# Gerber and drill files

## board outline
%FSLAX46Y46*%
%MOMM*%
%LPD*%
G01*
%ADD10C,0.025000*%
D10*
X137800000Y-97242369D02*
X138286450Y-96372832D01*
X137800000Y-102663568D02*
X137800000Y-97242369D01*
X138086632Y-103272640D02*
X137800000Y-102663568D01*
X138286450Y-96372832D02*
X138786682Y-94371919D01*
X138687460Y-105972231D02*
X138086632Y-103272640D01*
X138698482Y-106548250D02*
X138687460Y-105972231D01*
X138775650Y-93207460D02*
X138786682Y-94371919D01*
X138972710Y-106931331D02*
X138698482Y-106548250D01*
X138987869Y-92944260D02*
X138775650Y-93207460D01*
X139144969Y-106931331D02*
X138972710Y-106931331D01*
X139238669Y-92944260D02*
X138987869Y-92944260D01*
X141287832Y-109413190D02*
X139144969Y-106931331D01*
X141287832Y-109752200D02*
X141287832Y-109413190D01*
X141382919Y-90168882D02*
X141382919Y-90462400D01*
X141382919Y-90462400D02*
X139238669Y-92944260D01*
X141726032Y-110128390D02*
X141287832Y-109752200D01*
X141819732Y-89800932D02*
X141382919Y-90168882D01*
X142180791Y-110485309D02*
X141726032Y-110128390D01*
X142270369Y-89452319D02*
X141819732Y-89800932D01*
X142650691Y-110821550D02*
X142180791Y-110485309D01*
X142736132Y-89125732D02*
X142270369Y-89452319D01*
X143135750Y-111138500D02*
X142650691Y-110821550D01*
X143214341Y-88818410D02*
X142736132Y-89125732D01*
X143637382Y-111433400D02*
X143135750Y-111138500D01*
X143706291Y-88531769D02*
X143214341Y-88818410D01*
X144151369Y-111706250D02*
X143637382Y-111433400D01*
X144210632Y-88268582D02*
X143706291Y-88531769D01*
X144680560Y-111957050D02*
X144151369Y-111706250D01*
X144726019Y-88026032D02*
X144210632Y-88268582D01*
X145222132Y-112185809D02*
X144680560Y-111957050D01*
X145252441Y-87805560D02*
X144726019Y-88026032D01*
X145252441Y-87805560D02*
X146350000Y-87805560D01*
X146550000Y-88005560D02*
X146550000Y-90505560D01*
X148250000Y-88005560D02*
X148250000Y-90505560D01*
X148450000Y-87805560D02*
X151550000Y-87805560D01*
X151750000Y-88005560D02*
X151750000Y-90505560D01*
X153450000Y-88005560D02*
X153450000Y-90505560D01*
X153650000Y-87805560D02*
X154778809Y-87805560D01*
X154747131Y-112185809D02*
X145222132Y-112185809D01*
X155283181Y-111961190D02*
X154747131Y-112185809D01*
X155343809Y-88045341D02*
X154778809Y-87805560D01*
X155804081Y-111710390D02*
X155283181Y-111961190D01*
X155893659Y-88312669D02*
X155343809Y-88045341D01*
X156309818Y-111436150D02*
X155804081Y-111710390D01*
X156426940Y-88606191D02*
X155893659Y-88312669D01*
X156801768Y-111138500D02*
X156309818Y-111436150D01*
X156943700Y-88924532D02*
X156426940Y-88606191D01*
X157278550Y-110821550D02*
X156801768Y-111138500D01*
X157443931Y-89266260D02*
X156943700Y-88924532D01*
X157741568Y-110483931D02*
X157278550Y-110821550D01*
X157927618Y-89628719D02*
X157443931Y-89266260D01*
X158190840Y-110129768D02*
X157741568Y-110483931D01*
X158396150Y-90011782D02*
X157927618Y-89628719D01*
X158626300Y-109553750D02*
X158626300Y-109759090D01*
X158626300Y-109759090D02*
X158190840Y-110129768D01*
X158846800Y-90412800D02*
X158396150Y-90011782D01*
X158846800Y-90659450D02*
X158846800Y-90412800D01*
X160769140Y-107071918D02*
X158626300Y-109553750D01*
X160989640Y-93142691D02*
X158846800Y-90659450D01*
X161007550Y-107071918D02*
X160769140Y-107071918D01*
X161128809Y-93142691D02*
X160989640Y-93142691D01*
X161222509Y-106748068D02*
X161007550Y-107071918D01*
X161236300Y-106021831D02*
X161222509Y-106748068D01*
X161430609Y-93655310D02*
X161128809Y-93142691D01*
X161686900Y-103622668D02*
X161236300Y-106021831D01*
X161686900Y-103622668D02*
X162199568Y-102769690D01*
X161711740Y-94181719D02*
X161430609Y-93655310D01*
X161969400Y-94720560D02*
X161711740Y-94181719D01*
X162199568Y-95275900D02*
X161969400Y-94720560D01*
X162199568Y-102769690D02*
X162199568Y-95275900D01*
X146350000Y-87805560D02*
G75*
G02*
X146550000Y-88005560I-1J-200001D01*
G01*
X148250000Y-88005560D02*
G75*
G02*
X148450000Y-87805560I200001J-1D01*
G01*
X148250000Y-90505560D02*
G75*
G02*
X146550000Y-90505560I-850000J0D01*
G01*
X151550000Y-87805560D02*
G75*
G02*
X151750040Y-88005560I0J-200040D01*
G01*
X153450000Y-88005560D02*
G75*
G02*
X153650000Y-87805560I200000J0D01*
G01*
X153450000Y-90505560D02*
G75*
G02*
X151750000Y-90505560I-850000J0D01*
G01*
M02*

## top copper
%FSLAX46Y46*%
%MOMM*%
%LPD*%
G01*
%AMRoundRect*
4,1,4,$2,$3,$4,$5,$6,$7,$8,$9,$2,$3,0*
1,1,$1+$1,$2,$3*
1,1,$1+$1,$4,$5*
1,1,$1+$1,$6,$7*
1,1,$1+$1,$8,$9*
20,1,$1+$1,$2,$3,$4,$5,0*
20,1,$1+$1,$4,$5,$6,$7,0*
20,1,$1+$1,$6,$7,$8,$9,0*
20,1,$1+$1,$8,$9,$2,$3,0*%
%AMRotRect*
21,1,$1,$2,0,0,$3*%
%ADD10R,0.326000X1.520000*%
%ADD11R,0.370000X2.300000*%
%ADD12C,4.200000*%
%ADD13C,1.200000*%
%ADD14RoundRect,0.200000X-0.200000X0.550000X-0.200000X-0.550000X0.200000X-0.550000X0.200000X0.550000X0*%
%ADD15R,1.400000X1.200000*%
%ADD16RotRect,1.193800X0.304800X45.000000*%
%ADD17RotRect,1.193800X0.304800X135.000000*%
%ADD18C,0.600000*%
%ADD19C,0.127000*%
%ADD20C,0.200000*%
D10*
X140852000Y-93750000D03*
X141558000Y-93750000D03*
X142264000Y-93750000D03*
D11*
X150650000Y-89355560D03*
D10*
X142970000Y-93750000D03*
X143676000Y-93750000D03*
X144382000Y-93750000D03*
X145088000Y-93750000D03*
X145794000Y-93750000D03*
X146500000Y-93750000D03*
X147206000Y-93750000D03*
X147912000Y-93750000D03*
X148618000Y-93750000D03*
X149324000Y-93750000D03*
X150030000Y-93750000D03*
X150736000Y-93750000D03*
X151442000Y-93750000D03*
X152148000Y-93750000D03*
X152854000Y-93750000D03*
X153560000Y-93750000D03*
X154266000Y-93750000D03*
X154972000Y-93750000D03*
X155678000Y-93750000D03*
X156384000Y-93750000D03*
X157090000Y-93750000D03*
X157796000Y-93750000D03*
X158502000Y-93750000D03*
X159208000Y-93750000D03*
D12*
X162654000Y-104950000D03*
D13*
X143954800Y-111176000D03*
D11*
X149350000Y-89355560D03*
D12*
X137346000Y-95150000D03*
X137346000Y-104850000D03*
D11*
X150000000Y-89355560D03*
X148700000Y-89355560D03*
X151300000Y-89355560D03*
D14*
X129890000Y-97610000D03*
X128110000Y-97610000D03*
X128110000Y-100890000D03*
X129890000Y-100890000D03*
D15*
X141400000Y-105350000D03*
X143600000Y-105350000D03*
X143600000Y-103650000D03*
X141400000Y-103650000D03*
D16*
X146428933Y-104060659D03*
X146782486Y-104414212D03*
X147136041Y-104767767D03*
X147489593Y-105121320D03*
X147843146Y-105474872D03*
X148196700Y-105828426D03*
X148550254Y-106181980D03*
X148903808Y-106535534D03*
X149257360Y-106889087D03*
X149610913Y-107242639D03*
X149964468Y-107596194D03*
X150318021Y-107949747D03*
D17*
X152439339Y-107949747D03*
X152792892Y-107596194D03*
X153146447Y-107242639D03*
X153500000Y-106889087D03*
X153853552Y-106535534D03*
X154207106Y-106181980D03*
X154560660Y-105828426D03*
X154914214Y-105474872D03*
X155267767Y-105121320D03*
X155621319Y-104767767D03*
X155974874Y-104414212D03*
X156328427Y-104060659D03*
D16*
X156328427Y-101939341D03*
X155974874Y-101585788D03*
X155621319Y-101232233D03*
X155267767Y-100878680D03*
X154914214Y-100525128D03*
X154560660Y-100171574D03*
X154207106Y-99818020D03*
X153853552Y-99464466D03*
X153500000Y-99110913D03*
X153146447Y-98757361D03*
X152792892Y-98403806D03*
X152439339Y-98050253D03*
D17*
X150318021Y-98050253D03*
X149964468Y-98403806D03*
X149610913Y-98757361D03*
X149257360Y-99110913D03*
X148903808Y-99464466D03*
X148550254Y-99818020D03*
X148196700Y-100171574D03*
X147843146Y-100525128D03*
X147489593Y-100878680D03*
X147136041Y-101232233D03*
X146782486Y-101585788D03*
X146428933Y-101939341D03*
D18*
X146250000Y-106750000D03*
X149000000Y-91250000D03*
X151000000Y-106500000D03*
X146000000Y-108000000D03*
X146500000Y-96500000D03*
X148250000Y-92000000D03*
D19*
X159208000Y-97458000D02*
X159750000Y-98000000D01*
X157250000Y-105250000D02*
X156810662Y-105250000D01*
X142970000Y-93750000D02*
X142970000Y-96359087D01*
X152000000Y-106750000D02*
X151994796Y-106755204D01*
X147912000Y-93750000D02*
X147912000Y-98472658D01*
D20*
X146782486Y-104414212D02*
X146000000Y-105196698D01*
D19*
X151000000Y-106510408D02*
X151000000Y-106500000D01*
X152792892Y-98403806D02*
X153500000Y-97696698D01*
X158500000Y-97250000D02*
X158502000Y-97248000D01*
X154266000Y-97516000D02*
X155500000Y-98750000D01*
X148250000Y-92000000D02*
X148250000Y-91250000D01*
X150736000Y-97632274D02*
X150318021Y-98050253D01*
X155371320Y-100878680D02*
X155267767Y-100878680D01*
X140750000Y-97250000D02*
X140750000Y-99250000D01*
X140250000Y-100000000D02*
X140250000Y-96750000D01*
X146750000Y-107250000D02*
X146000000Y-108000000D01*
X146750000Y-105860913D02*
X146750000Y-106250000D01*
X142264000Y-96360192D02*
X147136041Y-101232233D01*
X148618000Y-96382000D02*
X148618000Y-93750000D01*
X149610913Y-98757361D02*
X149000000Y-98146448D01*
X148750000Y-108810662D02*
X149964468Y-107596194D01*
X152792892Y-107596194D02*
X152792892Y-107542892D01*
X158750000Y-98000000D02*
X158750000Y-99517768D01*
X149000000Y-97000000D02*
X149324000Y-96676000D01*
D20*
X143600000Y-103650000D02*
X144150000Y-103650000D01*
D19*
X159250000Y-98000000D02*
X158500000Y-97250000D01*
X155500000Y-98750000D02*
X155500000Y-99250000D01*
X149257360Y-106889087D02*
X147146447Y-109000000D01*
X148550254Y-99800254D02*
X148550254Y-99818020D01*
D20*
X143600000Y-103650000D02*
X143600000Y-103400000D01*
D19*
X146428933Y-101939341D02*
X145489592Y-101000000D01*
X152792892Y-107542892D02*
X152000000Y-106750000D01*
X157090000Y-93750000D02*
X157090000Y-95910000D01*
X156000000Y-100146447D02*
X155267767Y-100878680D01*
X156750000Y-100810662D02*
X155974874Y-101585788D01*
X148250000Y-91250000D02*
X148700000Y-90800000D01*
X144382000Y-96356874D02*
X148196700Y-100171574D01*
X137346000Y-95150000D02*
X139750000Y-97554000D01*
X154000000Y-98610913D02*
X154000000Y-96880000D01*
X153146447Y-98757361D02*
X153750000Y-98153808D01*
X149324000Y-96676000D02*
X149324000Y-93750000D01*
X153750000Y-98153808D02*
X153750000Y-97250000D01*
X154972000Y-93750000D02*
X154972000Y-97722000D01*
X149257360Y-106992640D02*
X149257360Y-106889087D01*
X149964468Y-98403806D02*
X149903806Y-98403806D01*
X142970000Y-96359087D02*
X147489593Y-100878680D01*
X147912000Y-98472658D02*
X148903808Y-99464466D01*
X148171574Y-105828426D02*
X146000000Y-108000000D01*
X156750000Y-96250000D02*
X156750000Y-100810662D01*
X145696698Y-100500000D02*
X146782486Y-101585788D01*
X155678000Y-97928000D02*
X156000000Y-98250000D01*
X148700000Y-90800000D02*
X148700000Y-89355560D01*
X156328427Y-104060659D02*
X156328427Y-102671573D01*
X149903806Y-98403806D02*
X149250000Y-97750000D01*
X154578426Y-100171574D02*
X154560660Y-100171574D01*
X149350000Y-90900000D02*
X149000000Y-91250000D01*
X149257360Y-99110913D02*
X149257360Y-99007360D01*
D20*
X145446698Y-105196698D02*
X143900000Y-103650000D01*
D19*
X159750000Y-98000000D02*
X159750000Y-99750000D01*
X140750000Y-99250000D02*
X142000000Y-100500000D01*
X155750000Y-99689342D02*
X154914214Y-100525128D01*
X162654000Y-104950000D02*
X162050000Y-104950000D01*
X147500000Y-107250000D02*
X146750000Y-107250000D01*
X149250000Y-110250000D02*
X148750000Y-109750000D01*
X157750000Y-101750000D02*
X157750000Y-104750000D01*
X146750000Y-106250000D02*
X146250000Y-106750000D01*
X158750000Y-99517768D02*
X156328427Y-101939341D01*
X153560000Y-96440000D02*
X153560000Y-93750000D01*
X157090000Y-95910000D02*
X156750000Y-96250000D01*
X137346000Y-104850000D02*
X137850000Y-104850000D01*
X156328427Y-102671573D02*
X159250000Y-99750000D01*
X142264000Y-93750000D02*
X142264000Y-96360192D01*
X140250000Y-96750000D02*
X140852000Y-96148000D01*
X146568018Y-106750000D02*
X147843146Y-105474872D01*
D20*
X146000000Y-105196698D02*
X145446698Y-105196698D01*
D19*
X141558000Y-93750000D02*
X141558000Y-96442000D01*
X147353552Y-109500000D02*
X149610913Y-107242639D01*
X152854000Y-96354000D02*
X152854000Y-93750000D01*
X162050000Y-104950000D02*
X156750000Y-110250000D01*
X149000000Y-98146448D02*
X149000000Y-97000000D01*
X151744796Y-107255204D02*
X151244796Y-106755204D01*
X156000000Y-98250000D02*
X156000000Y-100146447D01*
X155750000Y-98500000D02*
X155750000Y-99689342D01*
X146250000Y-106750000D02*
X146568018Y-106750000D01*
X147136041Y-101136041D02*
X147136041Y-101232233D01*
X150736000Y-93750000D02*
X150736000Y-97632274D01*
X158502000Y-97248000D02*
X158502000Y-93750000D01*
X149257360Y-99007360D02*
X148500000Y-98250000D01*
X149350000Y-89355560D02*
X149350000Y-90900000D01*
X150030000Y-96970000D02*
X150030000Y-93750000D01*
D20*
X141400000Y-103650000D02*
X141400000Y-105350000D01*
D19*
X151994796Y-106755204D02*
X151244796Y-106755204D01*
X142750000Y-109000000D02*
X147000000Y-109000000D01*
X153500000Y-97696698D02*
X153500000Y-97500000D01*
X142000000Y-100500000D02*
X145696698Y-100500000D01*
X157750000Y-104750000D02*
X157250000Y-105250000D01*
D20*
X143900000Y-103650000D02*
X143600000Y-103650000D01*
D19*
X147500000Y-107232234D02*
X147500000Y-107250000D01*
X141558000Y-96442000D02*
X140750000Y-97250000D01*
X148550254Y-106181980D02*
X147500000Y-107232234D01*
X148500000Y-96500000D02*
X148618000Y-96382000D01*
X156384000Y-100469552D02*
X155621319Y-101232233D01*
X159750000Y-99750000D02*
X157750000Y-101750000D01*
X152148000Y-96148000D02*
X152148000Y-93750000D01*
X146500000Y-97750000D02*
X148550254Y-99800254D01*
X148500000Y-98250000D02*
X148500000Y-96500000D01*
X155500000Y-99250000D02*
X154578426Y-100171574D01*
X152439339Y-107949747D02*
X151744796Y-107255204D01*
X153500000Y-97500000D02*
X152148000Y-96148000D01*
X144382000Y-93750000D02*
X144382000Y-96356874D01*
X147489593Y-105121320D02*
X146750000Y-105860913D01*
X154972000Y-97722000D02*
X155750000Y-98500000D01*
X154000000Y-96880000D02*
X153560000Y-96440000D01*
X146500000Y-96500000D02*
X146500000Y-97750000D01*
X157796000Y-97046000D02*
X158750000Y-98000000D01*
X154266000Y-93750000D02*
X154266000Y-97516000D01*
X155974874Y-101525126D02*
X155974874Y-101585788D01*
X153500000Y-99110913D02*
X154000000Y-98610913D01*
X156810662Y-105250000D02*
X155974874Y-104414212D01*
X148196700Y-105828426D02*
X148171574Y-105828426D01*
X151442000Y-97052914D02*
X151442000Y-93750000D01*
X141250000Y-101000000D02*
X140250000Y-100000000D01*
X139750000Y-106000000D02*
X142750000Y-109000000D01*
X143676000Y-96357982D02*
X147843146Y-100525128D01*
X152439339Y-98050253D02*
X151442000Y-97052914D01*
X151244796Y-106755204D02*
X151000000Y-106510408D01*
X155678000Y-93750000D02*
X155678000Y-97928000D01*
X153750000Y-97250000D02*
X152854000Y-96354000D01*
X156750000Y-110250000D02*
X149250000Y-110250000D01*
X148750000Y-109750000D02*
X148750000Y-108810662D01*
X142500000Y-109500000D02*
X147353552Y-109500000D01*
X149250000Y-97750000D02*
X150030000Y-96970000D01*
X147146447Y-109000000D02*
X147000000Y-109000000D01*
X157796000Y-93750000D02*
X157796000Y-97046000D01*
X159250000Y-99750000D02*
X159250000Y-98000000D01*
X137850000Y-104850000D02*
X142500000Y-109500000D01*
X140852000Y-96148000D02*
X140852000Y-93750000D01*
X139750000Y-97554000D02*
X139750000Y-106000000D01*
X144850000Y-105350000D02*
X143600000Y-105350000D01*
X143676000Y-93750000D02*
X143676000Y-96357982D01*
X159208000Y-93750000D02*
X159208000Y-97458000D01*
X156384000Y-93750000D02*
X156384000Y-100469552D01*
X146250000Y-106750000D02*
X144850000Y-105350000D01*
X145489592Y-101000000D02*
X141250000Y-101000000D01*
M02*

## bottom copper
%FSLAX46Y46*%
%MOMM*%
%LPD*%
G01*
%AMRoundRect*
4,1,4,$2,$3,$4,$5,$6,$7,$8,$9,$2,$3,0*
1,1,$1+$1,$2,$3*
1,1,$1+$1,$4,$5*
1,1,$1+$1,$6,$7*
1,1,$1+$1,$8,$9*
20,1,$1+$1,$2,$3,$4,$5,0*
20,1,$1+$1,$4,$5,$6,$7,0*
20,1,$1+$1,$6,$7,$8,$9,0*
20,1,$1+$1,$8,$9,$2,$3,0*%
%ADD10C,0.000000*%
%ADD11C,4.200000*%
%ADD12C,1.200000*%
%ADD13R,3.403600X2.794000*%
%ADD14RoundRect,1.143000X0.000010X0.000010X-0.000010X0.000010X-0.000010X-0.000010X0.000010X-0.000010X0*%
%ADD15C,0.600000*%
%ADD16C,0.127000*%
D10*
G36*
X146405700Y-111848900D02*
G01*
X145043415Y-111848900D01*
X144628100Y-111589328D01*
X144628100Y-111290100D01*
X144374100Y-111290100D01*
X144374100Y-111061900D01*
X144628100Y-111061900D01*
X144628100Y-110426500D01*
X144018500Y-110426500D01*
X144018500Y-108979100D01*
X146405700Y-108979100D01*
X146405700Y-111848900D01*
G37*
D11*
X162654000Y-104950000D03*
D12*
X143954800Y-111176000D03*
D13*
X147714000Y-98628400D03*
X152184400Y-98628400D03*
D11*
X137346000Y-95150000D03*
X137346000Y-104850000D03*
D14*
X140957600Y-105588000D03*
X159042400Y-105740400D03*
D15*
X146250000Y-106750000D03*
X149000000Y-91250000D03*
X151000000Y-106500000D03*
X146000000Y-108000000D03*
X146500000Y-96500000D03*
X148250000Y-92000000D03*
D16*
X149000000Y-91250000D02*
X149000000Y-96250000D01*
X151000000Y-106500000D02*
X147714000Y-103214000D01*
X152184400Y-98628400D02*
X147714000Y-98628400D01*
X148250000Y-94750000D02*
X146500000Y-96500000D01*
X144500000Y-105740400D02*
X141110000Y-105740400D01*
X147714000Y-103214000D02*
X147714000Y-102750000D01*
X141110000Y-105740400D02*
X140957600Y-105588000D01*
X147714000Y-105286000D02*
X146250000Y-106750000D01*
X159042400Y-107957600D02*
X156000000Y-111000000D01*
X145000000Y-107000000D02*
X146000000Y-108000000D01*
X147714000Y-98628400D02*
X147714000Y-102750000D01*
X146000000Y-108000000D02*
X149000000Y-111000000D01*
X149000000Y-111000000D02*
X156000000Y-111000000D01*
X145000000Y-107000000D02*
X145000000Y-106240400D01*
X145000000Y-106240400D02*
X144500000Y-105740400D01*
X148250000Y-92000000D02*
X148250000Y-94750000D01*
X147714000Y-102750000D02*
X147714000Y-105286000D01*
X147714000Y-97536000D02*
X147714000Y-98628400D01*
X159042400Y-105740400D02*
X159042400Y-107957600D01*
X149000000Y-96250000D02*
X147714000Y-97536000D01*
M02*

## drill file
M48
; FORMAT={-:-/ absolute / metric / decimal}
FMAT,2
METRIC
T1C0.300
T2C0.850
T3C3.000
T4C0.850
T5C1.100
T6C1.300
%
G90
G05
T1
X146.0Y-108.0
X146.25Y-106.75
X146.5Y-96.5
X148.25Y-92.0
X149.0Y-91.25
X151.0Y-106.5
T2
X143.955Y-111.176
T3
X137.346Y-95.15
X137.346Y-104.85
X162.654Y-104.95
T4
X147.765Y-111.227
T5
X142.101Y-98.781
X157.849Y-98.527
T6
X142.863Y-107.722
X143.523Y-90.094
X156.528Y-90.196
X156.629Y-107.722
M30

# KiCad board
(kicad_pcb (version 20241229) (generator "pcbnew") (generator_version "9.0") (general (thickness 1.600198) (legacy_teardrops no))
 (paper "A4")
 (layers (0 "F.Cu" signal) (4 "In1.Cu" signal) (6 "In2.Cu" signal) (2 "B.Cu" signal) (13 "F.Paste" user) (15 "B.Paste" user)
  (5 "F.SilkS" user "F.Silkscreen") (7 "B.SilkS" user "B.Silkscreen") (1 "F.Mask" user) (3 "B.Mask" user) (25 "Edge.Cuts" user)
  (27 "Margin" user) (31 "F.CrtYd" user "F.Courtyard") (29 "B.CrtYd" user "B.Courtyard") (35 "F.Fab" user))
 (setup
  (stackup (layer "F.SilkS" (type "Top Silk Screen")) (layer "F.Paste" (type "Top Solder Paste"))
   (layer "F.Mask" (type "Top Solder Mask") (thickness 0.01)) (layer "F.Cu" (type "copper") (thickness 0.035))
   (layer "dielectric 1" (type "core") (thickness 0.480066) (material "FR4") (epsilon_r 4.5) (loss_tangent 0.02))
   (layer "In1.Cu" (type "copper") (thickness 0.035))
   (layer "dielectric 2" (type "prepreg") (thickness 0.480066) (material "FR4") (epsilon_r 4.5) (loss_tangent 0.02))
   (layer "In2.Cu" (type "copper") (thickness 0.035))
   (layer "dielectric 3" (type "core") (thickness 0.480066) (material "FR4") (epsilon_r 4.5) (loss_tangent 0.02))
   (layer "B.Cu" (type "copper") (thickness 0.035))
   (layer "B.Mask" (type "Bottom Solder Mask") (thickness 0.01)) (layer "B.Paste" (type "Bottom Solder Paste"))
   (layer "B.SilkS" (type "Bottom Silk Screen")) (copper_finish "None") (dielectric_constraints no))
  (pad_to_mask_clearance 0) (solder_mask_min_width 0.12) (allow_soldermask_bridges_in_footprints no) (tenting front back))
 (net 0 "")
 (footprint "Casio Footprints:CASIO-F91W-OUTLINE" (layer "F.Cu") (at 150 100)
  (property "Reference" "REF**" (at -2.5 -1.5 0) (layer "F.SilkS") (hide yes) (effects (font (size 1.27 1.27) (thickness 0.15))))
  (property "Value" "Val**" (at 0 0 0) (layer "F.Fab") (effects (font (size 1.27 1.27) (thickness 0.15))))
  (fp_poly
   (pts (xy -3.5943 11.8489) (xy -4.956585 11.8489) (xy -5.3719 11.589328) (xy -5.3719 11.2901) (xy -5.6259 11.2901) (xy -5.6259 11.0619)
    (xy -5.3719 11.0619) (xy -5.3719 10.4265) (xy -5.9815 10.4265) (xy -5.9815 8.9791) (xy -3.5943 8.9791))
   (stroke (width 0) (type solid)) (fill yes) (layer "B.Cu"))
  (fp_line (start -12.2 -2.757631) (end -11.71355 -3.627168) (stroke (width 0.025) (type solid)) (layer "Edge.Cuts"))
  (fp_line (start -12.2 2.663568) (end -12.2 -2.757631) (stroke (width 0.025) (type solid)) (layer "Edge.Cuts"))
  (fp_line (start -11.913368 3.27264) (end -12.2 2.663568) (stroke (width 0.025) (type solid)) (layer "Edge.Cuts"))
  (fp_line (start -11.71355 -3.627168) (end -11.213318 -5.628081) (stroke (width 0.025) (type solid)) (layer "Edge.Cuts"))
  (fp_line (start -11.31254 5.972231) (end -11.913368 3.27264) (stroke (width 0.025) (type solid)) (layer "Edge.Cuts"))
  (fp_line (start -11.301518 6.54825) (end -11.31254 5.972231) (stroke (width 0.025) (type solid)) (layer "Edge.Cuts"))
  (fp_line (start -11.22435 -6.79254) (end -11.213318 -5.628081) (stroke (width 0.025) (type solid)) (layer "Edge.Cuts"))
  (fp_line (start -11.02729 6.931331) (end -11.301518 6.54825) (stroke (width 0.025) (type solid)) (layer "Edge.Cuts"))
  (fp_line (start -11.012131 -7.05574) (end -11.22435 -6.79254) (stroke (width 0.025) (type solid)) (layer "Edge.Cuts"))
  (fp_line (start -10.855031 6.931331) (end -11.02729 6.931331) (stroke (width 0.025) (type solid)) (layer "Edge.Cuts"))
  (fp_line (start -10.761331 -7.05574) (end -11.012131 -7.05574) (stroke (width 0.025) (type solid)) (layer "Edge.Cuts"))
  (fp_line (start -8.712168 9.41319) (end -10.855031 6.931331) (stroke (width 0.025) (type solid)) (layer "Edge.Cuts"))
  (fp_line (start -8.712168 9.7522) (end -8.712168 9.41319) (stroke (width 0.025) (type solid)) (layer "Edge.Cuts"))
  (fp_line (start -8.617081 -9.831118) (end -8.617081 -9.5376) (stroke (width 0.025) (type solid)) (layer "Edge.Cuts"))
  (fp_line (start -8.617081 -9.5376) (end -10.761331 -7.05574) (stroke (width 0.025) (type solid)) (layer "Edge.Cuts"))
  (fp_line (start -8.273968 10.12839) (end -8.712168 9.7522) (stroke (width 0.025) (type solid)) (layer "Edge.Cuts"))
  (fp_line (start -8.180268 -10.199068) (end -8.617081 -9.831118) (stroke (width 0.025) (type solid)) (layer "Edge.Cuts"))
  (fp_line (start -7.819209 10.485309) (end -8.273968 10.12839) (stroke (width 0.025) (type solid)) (layer "Edge.Cuts"))
  (fp_line (start -7.729631 -10.547681) (end -8.180268 -10.199068) (stroke (width 0.025) (type solid)) (layer "Edge.Cuts"))
  (fp_line (start -7.349309 10.82155) (end -7.819209 10.485309) (stroke (width 0.025) (type solid)) (layer "Edge.Cuts"))
  (fp_line (start -7.263868 -10.874268) (end -7.729631 -10.547681) (stroke (width 0.025) (type solid)) (layer "Edge.Cuts"))
  (fp_line (start -6.86425 11.1385) (end -7.349309 10.82155) (stroke (width 0.025) (type solid)) (layer "Edge.Cuts"))
  (fp_line (start -6.785659 -11.18159) (end -7.263868 -10.874268) (stroke (width 0.025) (type solid)) (layer "Edge.Cuts"))
  (fp_line (start -6.362618 11.4334) (end -6.86425 11.1385) (stroke (width 0.025) (type solid)) (layer "Edge.Cuts"))
  (fp_line (start -6.293709 -11.468231) (end -6.785659 -11.18159) (stroke (width 0.025) (type solid)) (layer "Edge.Cuts"))
  (fp_line (start -5.848631 11.70625) (end -6.362618 11.4334) (stroke (width 0.025) (type solid)) (layer "Edge.Cuts"))
  (fp_line (start -5.789368 -11.731418) (end -6.293709 -11.468231) (stroke (width 0.025) (type solid)) (layer "Edge.Cuts"))
  (fp_line (start -5.31944 11.95705) (end -5.848631 11.70625) (stroke (width 0.025) (type solid)) (layer "Edge.Cuts"))
  (fp_line (start -5.273981 -11.973968) (end -5.789368 -11.731418) (stroke (width 0.025) (type solid)) (layer "Edge.Cuts"))
  (fp_line (start -4.777868 12.185809) (end -5.31944 11.95705) (stroke (width 0.025) (type solid)) (layer "Edge.Cuts"))
  (fp_line (start -4.747559 -12.19444) (end -5.273981 -11.973968) (stroke (width 0.025) (type solid)) (layer "Edge.Cuts"))
  (fp_line (start -4.747559 -12.19444) (end -3.65 -12.19444) (stroke (width 0.025) (type solid)) (layer "Edge.Cuts"))
  (fp_line (start -3.45 -11.99444) (end -3.45 -9.49444) (stroke (width 0.025) (type solid)) (layer "Edge.Cuts"))
  (fp_line (start -1.75 -11.99444) (end -1.75 -9.49444) (stroke (width 0.025) (type solid)) (layer "Edge.Cuts"))
  (fp_line (start -1.55 -12.19444) (end 1.55 -12.19444) (stroke (width 0.025) (type solid)) (layer "Edge.Cuts"))
  (fp_line (start 1.75 -11.99444) (end 1.75 -9.49444) (stroke (width 0.025) (type solid)) (layer "Edge.Cuts"))
  (fp_line (start 3.45 -11.99444) (end 3.45 -9.49444) (stroke (width 0.025) (type solid)) (layer "Edge.Cuts"))
  (fp_line (start 3.65 -12.19444) (end 4.778809 -12.19444) (stroke (width 0.025) (type solid)) (layer "Edge.Cuts"))
  (fp_line (start 4.747131 12.185809) (end -4.777868 12.185809) (stroke (width 0.025) (type solid)) (layer "Edge.Cuts"))
  (fp_line (start 5.283181 11.96119) (end 4.747131 12.185809) (stroke (width 0.025) (type solid)) (layer "Edge.Cuts"))
  (fp_line (start 5.343809 -11.954659) (end 4.778809 -12.19444) (stroke (width 0.025) (type solid)) (layer "Edge.Cuts"))
  (fp_line (start 5.804081 11.71039) (end 5.283181 11.96119) (stroke (width 0.025) (type solid)) (layer "Edge.Cuts"))
  (fp_line (start 5.893659 -11.687331) (end 5.343809 -11.954659) (stroke (width 0.025) (type solid)) (layer "Edge.Cuts"))
  (fp_line (start 6.309818 11.43615) (end 5.804081 11.71039) (stroke (width 0.025) (type solid)) (layer "Edge.Cuts"))
  (fp_line (start 6.42694 -11.393809) (end 5.893659 -11.687331) (stroke (width 0.025) (type solid)) (layer "Edge.Cuts"))
  (fp_line (start 6.801768 11.1385) (end 6.309818 11.43615) (stroke (width 0.025) (type solid)) (layer "Edge.Cuts"))
  (fp_line (start 6.9437 -11.075468) (end 6.42694 -11.393809) (stroke (width 0.025) (type solid)) (layer "Edge.Cuts"))
  (fp_line (start 7.27855 10.82155) (end 6.801768 11.1385) (stroke (width 0.025) (type solid)) (layer "Edge.Cuts"))
  (fp_line (start 7.443931 -10.73374) (end 6.9437 -11.075468) (stroke (width 0.025) (type solid)) (layer "Edge.Cuts"))
  (fp_line (start 7.741568 10.483931) (end 7.27855 10.82155) (stroke (width 0.025) (type solid)) (layer "Edge.Cuts"))
  (fp_line (start 7.927618 -10.371281) (end 7.443931 -10.73374) (stroke (width 0.025) (type solid)) (layer "Edge.Cuts"))
  (fp_line (start 8.19084 10.129768) (end 7.741568 10.483931) (stroke (width 0.025) (type solid)) (layer "Edge.Cuts"))
  (fp_line (start 8.39615 -9.988218) (end 7.927618 -10.371281) (stroke (width 0.025) (type solid)) (layer "Edge.Cuts"))
  (fp_line (start 8.6263 9.55375) (end 8.6263 9.75909) (stroke (width 0.025) (type solid)) (layer "Edge.Cuts"))
  (fp_line (start 8.6263 9.75909) (end 8.19084 10.129768) (stroke (width 0.025) (type solid)) (layer "Edge.Cuts"))
  (fp_line (start 8.8468 -9.5872) (end 8.39615 -9.988218) (stroke (width 0.025) (type solid)) (layer "Edge.Cuts"))
  (fp_line (start 8.8468 -9.34055) (end 8.8468 -9.5872) (stroke (width 0.025) (type solid)) (layer "Edge.Cuts"))
  (fp_line (start 10.76914 7.071918) (end 8.6263 9.55375) (stroke (width 0.025) (type solid)) (layer "Edge.Cuts"))
  (fp_line (start 10.98964 -6.857309) (end 8.8468 -9.34055) (stroke (width 0.025) (type solid)) (layer "Edge.Cuts"))
  (fp_line (start 11.00755 7.071918) (end 10.76914 7.071918) (stroke (width 0.025) (type solid)) (layer "Edge.Cuts"))
  (fp_line (start 11.128809 -6.857309) (end 10.98964 -6.857309) (stroke (width 0.025) (type solid)) (layer "Edge.Cuts"))
  (fp_line (start 11.222509 6.748068) (end 11.00755 7.071918) (stroke (width 0.025) (type solid)) (layer "Edge.Cuts"))
  (fp_line (start 11.2363 6.021831) (end 11.222509 6.748068) (stroke (width 0.025) (type solid)) (layer "Edge.Cuts"))
  (fp_line (start 11.430609 -6.34469) (end 11.128809 -6.857309) (stroke (width 0.025) (type solid)) (layer "Edge.Cuts"))
  (fp_line (start 11.6869 3.622668) (end 11.2363 6.021831) (stroke (width 0.025) (type solid)) (layer "Edge.Cuts"))
  (fp_line (start 11.6869 3.622668) (end 12.199568 2.76969) (stroke (width 0.025) (type solid)) (layer "Edge.Cuts"))
  (fp_line (start 11.71174 -5.818281) (end 11.430609 -6.34469) (stroke (width 0.025) (type solid)) (layer "Edge.Cuts"))
  (fp_line (start 11.9694 -5.27944) (end 11.71174 -5.818281) (stroke (width 0.025) (type solid)) (layer "Edge.Cuts"))
  (fp_line (start 12.199568 -4.7241) (end 11.9694 -5.27944) (stroke (width 0.025) (type solid)) (layer "Edge.Cuts"))
  (fp_line (start 12.199568 2.76969) (end 12.199568 -4.7241) (stroke (width 0.025) (type solid)) (layer "Edge.Cuts"))
  (fp_arc (start -3.65 -12.19444) (mid -3.508579 -12.135861) (end -3.45 -11.99444) (stroke (width 0.025) (type solid)) (layer "Edge.Cuts"))
  (fp_arc (start -1.75 -11.99444) (mid -1.691421 -12.135861) (end -1.55 -12.19444) (stroke (width 0.025) (type solid)) (layer "Edge.Cuts"))
  (fp_arc (start -1.75 -9.49444) (mid -2.6 -8.64444) (end -3.45 -9.49444) (stroke (width 0.025) (type solid)) (layer "Edge.Cuts"))
  (fp_arc (start 1.55 -12.19444) (mid 1.691421 -12.135861) (end 1.75 -11.99444) (stroke (width 0.025) (type solid)) (layer "Edge.Cuts"))
  (fp_arc (start 3.45 -11.99444) (mid 3.508579 -12.135861) (end 3.65 -12.19444) (stroke (width 0.025) (type solid)) (layer "Edge.Cuts"))
  (fp_arc (start 3.45 -9.49444) (mid 2.6 -8.64444) (end 1.75 -9.49444) (stroke (width 0.025) (type solid)) (layer "Edge.Cuts"))
  (pad "" np_thru_hole circle (at -7.8994 -1.2192) (size 1.1 1.1) (drill 1.1) (layers "*.Cu" "*.Mask"))
  (pad "" np_thru_hole circle (at -7.1374 7.7216) (size 1.3 1.3) (drill 1.3) (layers "*.Cu" "*.Mask"))
  (pad "" np_thru_hole circle (at -6.477 -9.906) (size 1.3 1.3) (drill 1.3) (layers "*.Cu" "*.Mask"))
  (pad "" np_thru_hole circle (at -2.2352 11.2268) (size 0.85 0.85) (drill 0.85) (layers "*.Cu" "*.Mask"))
  (pad "" np_thru_hole circle (at 6.5278 -9.8044) (size 1.3 1.3) (drill 1.3) (layers "*.Cu" "*.Mask"))
  (pad "" np_thru_hole circle (at 6.6294 7.7216) (size 1.3 1.3) (drill 1.3) (layers "*.Cu" "*.Mask"))
  (pad "" np_thru_hole circle (at 7.8486 -1.4732) (size 1.1 1.1) (drill 1.1) (layers "*.Cu" "*.Mask"))
  (pad "1" smd rect (at -9.148 -6.25) (size 0.326 1.52) (layers "F.Cu" "F.Mask") (solder_mask_margin 0.0635))
  (pad "2" smd rect (at -8.442 -6.25) (size 0.326 1.52) (layers "F.Cu" "F.Mask") (solder_mask_margin 0.0635))
  (pad "3" smd rect (at -7.736 -6.25) (size 0.326 1.52) (layers "F.Cu" "F.Mask") (solder_mask_margin 0.0635))
  (pad "3V3" smd rect (at 0.65 -10.64444 90) (size 2.3 0.37) (layers "F.Cu" "F.Mask") (solder_mask_margin 0.0635))
  (pad "4" smd rect (at -7.03 -6.25) (size 0.326 1.52) (layers "F.Cu" "F.Mask") (solder_mask_margin 0.0635))
  (pad "5" smd rect (at -6.324 -6.25) (size 0.326 1.52) (layers "F.Cu" "F.Mask") (solder_mask_margin 0.0635))
  (pad "6" smd rect (at -5.618 -6.25) (size 0.326 1.52) (layers "F.Cu" "F.Mask") (solder_mask_margin 0.0635))
  (pad "7" smd rect (at -4.912 -6.25) (size 0.326 1.52) (layers "F.Cu" "F.Mask") (solder_mask_margin 0.0635))
  (pad "8" smd rect (at -4.206 -6.25) (size 0.326 1.52) (layers "F.Cu" "F.Mask") (solder_mask_margin 0.0635))
  (pad "9" smd rect (at -3.5 -6.25) (size 0.326 1.52) (layers "F.Cu" "F.Mask") (solder_mask_margin 0.0635))
  (pad "10" smd rect (at -2.794 -6.25) (size 0.326 1.52) (layers "F.Cu" "F.Mask") (solder_mask_margin 0.0635))
  (pad "11" smd rect (at -2.088 -6.25) (size 0.326 1.52) (layers "F.Cu" "F.Mask") (solder_mask_margin 0.0635))
  (pad "12" smd rect (at -1.382 -6.25) (size 0.326 1.52) (layers "F.Cu" "F.Mask") (solder_mask_margin 0.0635))
  (pad "13" smd rect (at -0.676 -6.25) (size 0.326 1.52) (layers "F.Cu" "F.Mask") (solder_mask_margin 0.0635))
  (pad "14" smd rect (at 0.03 -6.25) (size 0.326 1.52) (layers "F.Cu" "F.Mask") (solder_mask_margin 0.0635))
  (pad "15" smd rect (at 0.736 -6.25) (size 0.326 1.52) (layers "F.Cu" "F.Mask") (solder_mask_margin 0.0635))
  (pad "16" smd rect (at 1.442 -6.25) (size 0.326 1.52) (layers "F.Cu" "F.Mask") (solder_mask_margin 0.0635))
  (pad "17" smd rect (at 2.148 -6.25) (size 0.326 1.52) (layers "F.Cu" "F.Mask") (solder_mask_margin 0.0635))
  (pad "18" smd rect (at 2.854 -6.25) (size 0.326 1.52) (layers "F.Cu" "F.Mask") (solder_mask_margin 0.0635))
  (pad "19" smd rect (at 3.56 -6.25) (size 0.326 1.52) (layers "F.Cu" "F.Mask") (solder_mask_margin 0.0635))
  (pad "20" smd rect (at 4.266 -6.25) (size 0.326 1.52) (layers "F.Cu" "F.Mask") (solder_mask_margin 0.0635))
  (pad "21" smd rect (at 4.972 -6.25) (size 0.326 1.52) (layers "F.Cu" "F.Mask") (solder_mask_margin 0.0635))
  (pad "22" smd rect (at 5.678 -6.25) (size 0.326 1.52) (layers "F.Cu" "F.Mask") (solder_mask_margin 0.0635))
  (pad "23" smd rect (at 6.384 -6.25) (size 0.326 1.52) (layers "F.Cu" "F.Mask") (solder_mask_margin 0.0635))
  (pad "24" smd rect (at 7.09 -6.25) (size 0.326 1.52) (layers "F.Cu" "F.Mask") (solder_mask_margin 0.0635))
  (pad "25" smd rect (at 7.796 -6.25) (size 0.326 1.52) (layers "F.Cu" "F.Mask") (solder_mask_margin 0.0635))
  (pad "26" smd rect (at 8.502 -6.25) (size 0.326 1.52) (layers "F.Cu" "F.Mask") (solder_mask_margin 0.0635))
  (pad "27" smd rect (at 9.208 -6.25) (size 0.326 1.52) (layers "F.Cu" "F.Mask") (solder_mask_margin 0.0635))
  (pad "ALARM" thru_hole circle (at 12.654 4.95) (size 4.2 4.2) (drill 3) (layers "*.Cu" "*.Mask") (remove_unused_layers no)
   (solder_mask_margin 0.0635))
  (pad "BUZZER" thru_hole circle (at -6.0452 11.176) (size 1.2 1.2) (drill 0.85) (layers "*.Cu" "*.Mask") (remove_unused_layers no)
   (solder_mask_margin 0.0635))
  (pad "GND" smd rect (at -0.65 -10.64444 90) (size 2.3 0.37) (layers "F.Cu" "F.Mask") (solder_mask_margin 0.0635))
  (pad "GND1" smd rect (at -2.286 -1.3716 180) (size 3.4036 2.794) (layers "B.Cu" "B.Mask") (solder_mask_margin 0.0635) (zone_connect 2))
  (pad "GND2" smd rect (at 2.1844 -1.3716 180) (size 3.4036 2.794) (layers "B.Cu" "B.Mask") (solder_mask_margin 0.0635) (zone_connect 2))
  (pad "LIGHT" thru_hole circle (at -12.654 -4.85) (size 4.2 4.2) (drill 3) (layers "*.Cu" "*.Mask") (remove_unused_layers no)
   (solder_mask_margin 0.0635))
  (pad "MODE" thru_hole circle (at -12.654 4.85) (size 4.2 4.2) (drill 3) (layers "*.Cu" "*.Mask") (remove_unused_layers no)
   (solder_mask_margin 0.0635))
  (pad "SWCKJ" smd rect (at 0 -10.64444 90) (size 2.3 0.37) (layers "F.Cu" "F.Mask") (solder_mask_margin 0.0635))
  (pad "SWIM" smd rect (at -1.3 -10.64444 90) (size 2.3 0.37) (layers "F.Cu" "F.Mask") (solder_mask_margin 0.0635))
  (pad "UNUSED" smd rect (at 1.3 -10.64444 90) (size 2.3 0.37) (layers "F.Cu" "F.Mask") (solder_mask_margin 0.0635))
  (pad "VCC1" smd roundrect (at -9.0424 5.588 180) (size 2.286 2.286) (layers "B.Cu" "B.Mask") (roundrect_rratio 0.5)
   (solder_mask_margin 0.0635))
  (pad "VCC2" smd roundrect (at 9.0424 5.7404 180) (size 2.286 2.286) (layers "B.Cu" "B.Mask") (roundrect_rratio 0.5)
   (solder_mask_margin 0.0635)))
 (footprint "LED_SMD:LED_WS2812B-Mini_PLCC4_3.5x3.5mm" (layer "F.Cu") (at 129 99.25 -90)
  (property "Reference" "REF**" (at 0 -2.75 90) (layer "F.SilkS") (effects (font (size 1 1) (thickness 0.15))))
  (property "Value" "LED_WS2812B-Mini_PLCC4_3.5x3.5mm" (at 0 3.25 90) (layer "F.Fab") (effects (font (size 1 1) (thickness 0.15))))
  (pad "1" smd roundrect (at -1.64 -0.89 270) (size 1.5 0.8) (layers "F.Cu" "F.Mask" "F.Paste") (roundrect_rratio 0.25))
  (pad "2" smd roundrect (at -1.64 0.89 270) (size 1.5 0.8) (layers "F.Cu" "F.Mask" "F.Paste") (roundrect_rratio 0.25))
  (pad "3" smd roundrect (at 1.64 0.89 270) (size 1.5 0.8) (layers "F.Cu" "F.Mask" "F.Paste") (roundrect_rratio 0.25))
  (pad "4" smd roundrect (at 1.64 -0.89 270) (size 1.5 0.8) (layers "F.Cu" "F.Mask" "F.Paste") (roundrect_rratio 0.25)))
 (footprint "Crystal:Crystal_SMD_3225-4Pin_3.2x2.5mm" (layer "F.Cu") (at 142.5 104.5)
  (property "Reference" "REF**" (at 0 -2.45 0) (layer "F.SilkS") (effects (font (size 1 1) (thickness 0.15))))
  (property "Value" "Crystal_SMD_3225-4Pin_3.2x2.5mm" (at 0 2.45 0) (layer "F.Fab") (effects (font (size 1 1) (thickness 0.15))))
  (pad "1" smd rect (at -1.1 0.85) (size 1.4 1.2) (layers "F.Cu" "F.Mask" "F.Paste"))
  (pad "2" smd rect (at 1.1 0.85) (size 1.4 1.2) (layers "F.Cu" "F.Mask" "F.Paste"))
  (pad "3" smd rect (at 1.1 -0.85) (size 1.4 1.2) (layers "F.Cu" "F.Mask" "F.Paste"))
  (pad "4" smd rect (at -1.1 -0.85) (size 1.4 1.2) (layers "F.Cu" "F.Mask" "F.Paste")))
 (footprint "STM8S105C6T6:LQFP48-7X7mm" (layer "F.Cu") (at 151.37868 103 45)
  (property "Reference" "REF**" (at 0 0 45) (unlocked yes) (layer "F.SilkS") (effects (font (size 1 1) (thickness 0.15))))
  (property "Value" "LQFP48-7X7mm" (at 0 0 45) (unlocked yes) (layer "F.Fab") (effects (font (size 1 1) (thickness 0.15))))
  (pad "1" smd rect (at -4.249999 -2.75 45) (size 1.1938 0.3048) (layers "F.Cu" "F.Mask" "F.Paste"))
  (pad "2" smd rect (at -4.249999 -2.250001 45) (size 1.1938 0.3048) (layers "F.Cu" "F.Mask" "F.Paste"))
  (pad "3" smd rect (at -4.249999 -1.749999 45) (size 1.1938 0.3048) (layers "F.Cu" "F.Mask" "F.Paste"))
  (pad "4" smd rect (at -4.25 -1.25 45) (size 1.1938 0.3048) (layers "F.Cu" "F.Mask" "F.Paste"))
  (pad "5" smd rect (at -4.249999 -0.750001 45) (size 1.1938 0.3048) (layers "F.Cu" "F.Mask" "F.Paste"))
  (pad "6" smd rect (at -4.249999 -0.25 45) (size 1.1938 0.3048) (layers "F.Cu" "F.Mask" "F.Paste"))
  (pad "7" smd rect (at -4.249999 0.25 45) (size 1.1938 0.3048) (layers "F.Cu" "F.Mask" "F.Paste"))
  (pad "8" smd rect (at -4.249999 0.750001 45) (size 1.1938 0.3048) (layers "F.Cu" "F.Mask" "F.Paste"))
  (pad "9" smd rect (at -4.25 1.25 45) (size 1.1938 0.3048) (layers "F.Cu" "F.Mask" "F.Paste"))
  (pad "10" smd rect (at -4.249999 1.749999 45) (size 1.1938 0.3048) (layers "F.Cu" "F.Mask" "F.Paste"))
  (pad "11" smd rect (at -4.249999 2.250001 45) (size 1.1938 0.3048) (layers "F.Cu" "F.Mask" "F.Paste"))
  (pad "12" smd rect (at -4.249999 2.75 45) (size 1.1938 0.3048) (layers "F.Cu" "F.Mask" "F.Paste"))
  (pad "13" smd rect (at -2.75 4.249999 135) (size 1.1938 0.3048) (layers "F.Cu" "F.Mask" "F.Paste"))
  (pad "14" smd rect (at -2.250001 4.249999 135) (size 1.1938 0.3048) (layers "F.Cu" "F.Mask" "F.Paste"))
  (pad "15" smd rect (at -1.749999 4.249999 135) (size 1.1938 0.3048) (layers "F.Cu" "F.Mask" "F.Paste"))
  (pad "16" smd rect (at -1.25 4.25 135) (size 1.1938 0.3048) (layers "F.Cu" "F.Mask" "F.Paste"))
  (pad "17" smd rect (at -0.750001 4.249999 135) (size 1.1938 0.3048) (layers "F.Cu" "F.Mask" "F.Paste"))
  (pad "18" smd rect (at -0.25 4.249999 135) (size 1.1938 0.3048) (layers "F.Cu" "F.Mask" "F.Paste"))
  (pad "19" smd rect (at 0.25 4.249999 135) (size 1.1938 0.3048) (layers "F.Cu" "F.Mask" "F.Paste"))
  (pad "20" smd rect (at 0.750001 4.249999 135) (size 1.1938 0.3048) (layers "F.Cu" "F.Mask" "F.Paste"))
  (pad "21" smd rect (at 1.25 4.25 135) (size 1.1938 0.3048) (layers "F.Cu" "F.Mask" "F.Paste"))
  (pad "22" smd rect (at 1.749999 4.249999 135) (size 1.1938 0.3048) (layers "F.Cu" "F.Mask" "F.Paste"))
  (pad "23" smd rect (at 2.250001 4.249999 135) (size 1.1938 0.3048) (layers "F.Cu" "F.Mask" "F.Paste"))
  (pad "24" smd rect (at 2.75 4.249999 135) (size 1.1938 0.3048) (layers "F.Cu" "F.Mask" "F.Paste"))
  (pad "25" smd rect (at 4.249999 2.75 45) (size 1.1938 0.3048) (layers "F.Cu" "F.Mask" "F.Paste"))
  (pad "26" smd rect (at 4.249999 2.250001 45) (size 1.1938 0.3048) (layers "F.Cu" "F.Mask" "F.Paste"))
  (pad "27" smd rect (at 4.249999 1.749999 45) (size 1.1938 0.3048) (layers "F.Cu" "F.Mask" "F.Paste"))
  (pad "28" smd rect (at 4.25 1.25 45) (size 1.1938 0.3048) (layers "F.Cu" "F.Mask" "F.Paste"))
  (pad "29" smd rect (at 4.249999 0.750001 45) (size 1.1938 0.3048) (layers "F.Cu" "F.Mask" "F.Paste"))
  (pad "30" smd rect (at 4.249999 0.25 45) (size 1.1938 0.3048) (layers "F.Cu" "F.Mask" "F.Paste"))
  (pad "31" smd rect (at 4.249999 -0.25 45) (size 1.1938 0.3048) (layers "F.Cu" "F.Mask" "F.Paste"))
  (pad "32" smd rect (at 4.249999 -0.750001 45) (size 1.1938 0.3048) (layers "F.Cu" "F.Mask" "F.Paste"))
  (pad "33" smd rect (at 4.25 -1.25 45) (size 1.1938 0.3048) (layers "F.Cu" "F.Mask" "F.Paste"))
  (pad "34" smd rect (at 4.249999 -1.749999 45) (size 1.1938 0.3048) (layers "F.Cu" "F.Mask" "F.Paste"))
  (pad "35" smd rect (at 4.249999 -2.250001 45) (size 1.1938 0.3048) (layers "F.Cu" "F.Mask" "F.Paste"))
  (pad "36" smd rect (at 4.249999 -2.75 45) (size 1.1938 0.3048) (layers "F.Cu" "F.Mask" "F.Paste"))
  (pad "37" smd rect (at 2.75 -4.249999 135) (size 1.1938 0.3048) (layers "F.Cu" "F.Mask" "F.Paste"))
  (pad "38" smd rect (at 2.250001 -4.249999 135) (size 1.1938 0.3048) (layers "F.Cu" "F.Mask" "F.Paste"))
  (pad "39" smd rect (at 1.749999 -4.249999 135) (size 1.1938 0.3048) (layers "F.Cu" "F.Mask" "F.Paste"))
  (pad "40" smd rect (at 1.25 -4.25 135) (size 1.1938 0.3048) (layers "F.Cu" "F.Mask" "F.Paste"))
  (pad "41" smd rect (at 0.750001 -4.249999 135) (size 1.1938 0.3048) (layers "F.Cu" "F.Mask" "F.Paste"))
  (pad "42" smd rect (at 0.25 -4.249999 135) (size 1.1938 0.3048) (layers "F.Cu" "F.Mask" "F.Paste"))
  (pad "43" smd rect (at -0.25 -4.249999 135) (size 1.1938 0.3048) (layers "F.Cu" "F.Mask" "F.Paste"))
  (pad "44" smd rect (at -0.750001 -4.249999 135) (size 1.1938 0.3048) (layers "F.Cu" "F.Mask" "F.Paste"))
  (pad "45" smd rect (at -1.25 -4.25 135) (size 1.1938 0.3048) (layers "F.Cu" "F.Mask" "F.Paste"))
  (pad "46" smd rect (at -1.749999 -4.249999 135) (size 1.1938 0.3048) (layers "F.Cu" "F.Mask" "F.Paste"))
  (pad "47" smd rect (at -2.250001 -4.249999 135) (size 1.1938 0.3048) (layers "F.Cu" "F.Mask" "F.Paste"))
  (pad "48" smd rect (at -2.75 -4.249999 135) (size 1.1938 0.3048) (layers "F.Cu" "F.Mask" "F.Paste")))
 (segment (start 159.208 97.458) (end 159.75 98) (width 0.127) (layer "F.Cu") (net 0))
 (segment (start 157.25 105.25) (end 156.810662 105.25) (width 0.127) (layer "F.Cu") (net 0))
 (segment (start 142.97 93.75) (end 142.97 96.359087) (width 0.127) (layer "F.Cu") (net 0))
 (segment (start 152 106.75) (end 151.994796 106.755204) (width 0.127) (layer "F.Cu") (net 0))
 (segment (start 147.912 93.75) (end 147.912 98.472658) (width 0.127) (layer "F.Cu") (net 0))
 (segment (start 146.782486 104.414212) (end 146 105.196698) (width 0.2) (layer "F.Cu") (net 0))
 (segment (start 151 106.510408) (end 151 106.5) (width 0.127) (layer "F.Cu") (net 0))
 (segment (start 152.792892 98.403806) (end 153.5 97.696698) (width 0.127) (layer "F.Cu") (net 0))
 (segment (start 158.5 97.25) (end 158.502 97.248) (width 0.127) (layer "F.Cu") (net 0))
 (segment (start 154.266 97.516) (end 155.5 98.75) (width 0.127) (layer "F.Cu") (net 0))
 (segment (start 148.25 92) (end 148.25 91.25) (width 0.127) (layer "F.Cu") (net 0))
 (segment (start 150.736 97.632274) (end 150.318021 98.050253) (width 0.127) (layer "F.Cu") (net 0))
 (segment (start 155.37132 100.87868) (end 155.267767 100.87868) (width 0.127) (layer "F.Cu") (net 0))
 (segment (start 140.75 97.25) (end 140.75 99.25) (width 0.127) (layer "F.Cu") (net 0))
 (segment (start 140.25 100) (end 140.25 96.75) (width 0.127) (layer "F.Cu") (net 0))
 (segment (start 146.75 107.25) (end 146 108) (width 0.127) (layer "F.Cu") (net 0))
 (segment (start 146.75 105.860913) (end 146.75 106.25) (width 0.127) (layer "F.Cu") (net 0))
 (segment (start 142.264 96.360192) (end 147.136041 101.232233) (width 0.127) (layer "F.Cu") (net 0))
 (segment (start 148.618 96.382) (end 148.618 93.75) (width 0.127) (layer "F.Cu") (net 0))
 (segment (start 149.610913 98.757361) (end 149 98.146448) (width 0.127) (layer "F.Cu") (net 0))
 (segment (start 148.75 108.810662) (end 149.964468 107.596194) (width 0.127) (layer "F.Cu") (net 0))
 (segment (start 152.792892 107.596194) (end 152.792892 107.542892) (width 0.127) (layer "F.Cu") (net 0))
 (segment (start 158.75 98) (end 158.75 99.517768) (width 0.127) (layer "F.Cu") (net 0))
 (segment (start 149 97) (end 149.324 96.676) (width 0.127) (layer "F.Cu") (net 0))
 (segment (start 143.6 103.65) (end 144.15 103.65) (width 0.2) (layer "F.Cu") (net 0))
 (segment (start 159.25 98) (end 158.5 97.25) (width 0.127) (layer "F.Cu") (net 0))
 (segment (start 155.5 98.75) (end 155.5 99.25) (width 0.127) (layer "F.Cu") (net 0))
 (segment (start 149.25736 106.889087) (end 147.146447 109) (width 0.127) (layer "F.Cu") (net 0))
 (segment (start 148.550254 99.800254) (end 148.550254 99.81802) (width 0.127) (layer "F.Cu") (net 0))
 (segment (start 143.6 103.65) (end 143.6 103.4) (width 0.2) (layer "F.Cu") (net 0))
 (segment (start 146.428933 101.939341) (end 145.489592 101) (width 0.127) (layer "F.Cu") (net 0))
 (segment (start 152.792892 107.542892) (end 152 106.75) (width 0.127) (layer "F.Cu") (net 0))
 (segment (start 157.09 93.75) (end 157.09 95.91) (width 0.127) (layer "F.Cu") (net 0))
 (segment (start 156 100.146447) (end 155.267767 100.87868) (width 0.127) (layer "F.Cu") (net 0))
 (segment (start 156.75 100.810662) (end 155.974874 101.585788) (width 0.127) (layer "F.Cu") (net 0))
 (segment (start 148.25 91.25) (end 148.7 90.8) (width 0.127) (layer "F.Cu") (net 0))
 (segment (start 144.382 96.356874) (end 148.1967 100.171574) (width 0.127) (layer "F.Cu") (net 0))
 (segment (start 137.346 95.15) (end 139.75 97.554) (width 0.127) (layer "F.Cu") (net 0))
 (segment (start 154 98.610913) (end 154 96.88) (width 0.127) (layer "F.Cu") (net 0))
 (segment (start 153.146447 98.757361) (end 153.75 98.153808) (width 0.127) (layer "F.Cu") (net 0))
 (segment (start 149.324 96.676) (end 149.324 93.75) (width 0.127) (layer "F.Cu") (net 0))
 (segment (start 153.75 98.153808) (end 153.75 97.25) (width 0.127) (layer "F.Cu") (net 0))
 (segment (start 154.972 93.75) (end 154.972 97.722) (width 0.127) (layer "F.Cu") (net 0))
 (segment (start 149.25736 106.99264) (end 149.25736 106.889087) (width 0.127) (layer "F.Cu") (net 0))
 (segment (start 149.964468 98.403806) (end 149.903806 98.403806) (width 0.127) (layer "F.Cu") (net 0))
 (segment (start 142.97 96.359087) (end 147.489593 100.87868) (width 0.127) (layer "F.Cu") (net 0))
 (segment (start 147.912 98.472658) (end 148.903808 99.464466) (width 0.127) (layer "F.Cu") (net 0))
 (segment (start 148.171574 105.828426) (end 146 108) (width 0.127) (layer "F.Cu") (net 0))
 (segment (start 156.75 96.25) (end 156.75 100.810662) (width 0.127) (layer "F.Cu") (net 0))
 (segment (start 145.696698 100.5) (end 146.782486 101.585788) (width 0.127) (layer "F.Cu") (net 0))
 (segment (start 155.678 97.928) (end 156 98.25) (width 0.127) (layer "F.Cu") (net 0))
 (segment (start 148.7 90.8) (end 148.7 89.35556) (width 0.127) (layer "F.Cu") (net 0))
 (segment (start 156.328427 104.060659) (end 156.328427 102.671573) (width 0.127) (layer "F.Cu") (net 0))
 (segment (start 149.903806 98.403806) (end 149.25 97.75) (width 0.127) (layer "F.Cu") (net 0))
 (segment (start 154.578426 100.171574) (end 154.56066 100.171574) (width 0.127) (layer "F.Cu") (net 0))
 (segment (start 149.35 90.9) (end 149 91.25) (width 0.127) (layer "F.Cu") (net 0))
 (segment (start 149.25736 99.110913) (end 149.25736 99.00736) (width 0.127) (layer "F.Cu") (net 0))
 (segment (start 145.446698 105.196698) (end 143.9 103.65) (width 0.2) (layer "F.Cu") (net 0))
 (segment (start 159.75 98) (end 159.75 99.75) (width 0.127) (layer "F.Cu") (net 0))
 (segment (start 140.75 99.25) (end 142 100.5) (width 0.127) (layer "F.Cu") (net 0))
 (segment (start 155.75 99.689342) (end 154.914214 100.525128) (width 0.127) (layer "F.Cu") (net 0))
 (segment (start 162.654 104.95) (end 162.05 104.95) (width 0.127) (layer "F.Cu") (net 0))
 (segment (start 147.5 107.25) (end 146.75 107.25) (width 0.127) (layer "F.Cu") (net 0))
 (segment (start 149.25 110.25) (end 148.75 109.75) (width 0.127) (layer "F.Cu") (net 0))
 (segment (start 157.75 101.75) (end 157.75 104.75) (width 0.127) (layer "F.Cu") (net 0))
 (segment (start 146.75 106.25) (end 146.25 106.75) (width 0.127) (layer "F.Cu") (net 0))
 (segment (start 158.75 99.517768) (end 156.328427 101.939341) (width 0.127) (layer "F.Cu") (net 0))
 (segment (start 153.56 96.44) (end 153.56 93.75) (width 0.127) (layer "F.Cu") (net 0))
 (segment (start 157.09 95.91) (end 156.75 96.25) (width 0.127) (layer "F.Cu") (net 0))
 (segment (start 137.346 104.85) (end 137.85 104.85) (width 0.127) (layer "F.Cu") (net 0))
 (segment (start 156.328427 102.671573) (end 159.25 99.75) (width 0.127) (layer "F.Cu") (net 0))
 (segment (start 142.264 93.75) (end 142.264 96.360192) (width 0.127) (layer "F.Cu") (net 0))
 (segment (start 140.25 96.75) (end 140.852 96.148) (width 0.127) (layer "F.Cu") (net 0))
 (segment (start 146.568018 106.75) (end 147.843146 105.474872) (width 0.127) (layer "F.Cu") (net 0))
 (segment (start 146 105.196698) (end 145.446698 105.196698) (width 0.2) (layer "F.Cu") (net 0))
 (segment (start 141.558 93.75) (end 141.558 96.442) (width 0.127) (layer "F.Cu") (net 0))
 (segment (start 147.353552 109.5) (end 149.610913 107.242639) (width 0.127) (layer "F.Cu") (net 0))
 (segment (start 152.854 96.354) (end 152.854 93.75) (width 0.127) (layer "F.Cu") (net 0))
 (segment (start 162.05 104.95) (end 156.75 110.25) (width 0.127) (layer "F.Cu") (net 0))
 (segment (start 149 98.146448) (end 149 97) (width 0.127) (layer "F.Cu") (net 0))
 (segment (start 151.744796 107.255204) (end 151.244796 106.755204) (width 0.127) (layer "F.Cu") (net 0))
 (segment (start 156 98.25) (end 156 100.146447) (width 0.127) (layer "F.Cu") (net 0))
 (segment (start 155.75 98.5) (end 155.75 99.689342) (width 0.127) (layer "F.Cu") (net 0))
 (segment (start 146.25 106.75) (end 146.568018 106.75) (width 0.127) (layer "F.Cu") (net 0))
 (segment (start 147.136041 101.136041) (end 147.136041 101.232233) (width 0.127) (layer "F.Cu") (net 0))
 (segment (start 150.736 93.75) (end 150.736 97.632274) (width 0.127) (layer "F.Cu") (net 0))
 (segment (start 158.502 97.248) (end 158.502 93.75) (width 0.127) (layer "F.Cu") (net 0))
 (segment (start 149.25736 99.00736) (end 148.5 98.25) (width 0.127) (layer "F.Cu") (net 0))
 (segment (start 149.35 89.35556) (end 149.35 90.9) (width 0.127) (layer "F.Cu") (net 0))
 (segment (start 150.03 96.97) (end 150.03 93.75) (width 0.127) (layer "F.Cu") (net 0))
 (segment (start 141.4 103.65) (end 141.4 105.35) (width 0.2) (layer "F.Cu") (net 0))
 (segment (start 151.994796 106.755204) (end 151.244796 106.755204) (width 0.127) (layer "F.Cu") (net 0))
 (segment (start 142.75 109) (end 147 109) (width 0.127) (layer "F.Cu") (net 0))
 (segment (start 153.5 97.696698) (end 153.5 97.5) (width 0.127) (layer "F.Cu") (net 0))
 (segment (start 142 100.5) (end 145.696698 100.5) (width 0.127) (layer "F.Cu") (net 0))
 (segment (start 157.75 104.75) (end 157.25 105.25) (width 0.127) (layer "F.Cu") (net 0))
 (segment (start 143.9 103.65) (end 143.6 103.65) (width 0.2) (layer "F.Cu") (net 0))
 (segment (start 147.5 107.232234) (end 147.5 107.25) (width 0.127) (layer "F.Cu") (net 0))
 (segment (start 141.558 96.442) (end 140.75 97.25) (width 0.127) (layer "F.Cu") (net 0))
 (segment (start 148.550254 106.18198) (end 147.5 107.232234) (width 0.127) (layer "F.Cu") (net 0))
 (segment (start 148.5 96.5) (end 148.618 96.382) (width 0.127) (layer "F.Cu") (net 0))
 (segment (start 156.384 100.469552) (end 155.621319 101.232233) (width 0.127) (layer "F.Cu") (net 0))
 (segment (start 159.75 99.75) (end 157.75 101.75) (width 0.127) (layer "F.Cu") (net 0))
 (segment (start 152.148 96.148) (end 152.148 93.75) (width 0.127) (layer "F.Cu") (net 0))
 (segment (start 146.5 97.75) (end 148.550254 99.800254) (width 0.127) (layer "F.Cu") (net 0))
 (segment (start 148.5 98.25) (end 148.5 96.5) (width 0.127) (layer "F.Cu") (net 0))
 (segment (start 155.5 99.25) (end 154.578426 100.171574) (width 0.127) (layer "F.Cu") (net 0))
 (segment (start 152.439339 107.949747) (end 151.744796 107.255204) (width 0.127) (layer "F.Cu") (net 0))
 (segment (start 153.5 97.5) (end 152.148 96.148) (width 0.127) (layer "F.Cu") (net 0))
 (segment (start 144.382 93.75) (end 144.382 96.356874) (width 0.127) (layer "F.Cu") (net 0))
 (segment (start 147.489593 105.12132) (end 146.75 105.860913) (width 0.127) (layer "F.Cu") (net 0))
 (segment (start 154.972 97.722) (end 155.75 98.5) (width 0.127) (layer "F.Cu") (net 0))
 (segment (start 154 96.88) (end 153.56 96.44) (width 0.127) (layer "F.Cu") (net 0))
 (segment (start 146.5 96.5) (end 146.5 97.75) (width 0.127) (layer "F.Cu") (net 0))
 (segment (start 157.796 97.046) (end 158.75 98) (width 0.127) (layer "F.Cu") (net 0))
 (segment (start 154.266 93.75) (end 154.266 97.516) (width 0.127) (layer "F.Cu") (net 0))
 (segment (start 155.974874 101.525126) (end 155.974874 101.585788) (width 0.127) (layer "F.Cu") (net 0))
 (segment (start 153.5 99.110913) (end 154 98.610913) (width 0.127) (layer "F.Cu") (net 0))
 (segment (start 156.810662 105.25) (end 155.974874 104.414212) (width 0.127) (layer "F.Cu") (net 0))
 (segment (start 148.1967 105.828426) (end 148.171574 105.828426) (width 0.127) (layer "F.Cu") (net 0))
 (segment (start 151.442 97.052914) (end 151.442 93.75) (width 0.127) (layer "F.Cu") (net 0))
 (segment (start 141.25 101) (end 140.25 100) (width 0.127) (layer "F.Cu") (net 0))
 (segment (start 139.75 106) (end 142.75 109) (width 0.127) (layer "F.Cu") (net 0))
 (segment (start 143.676 96.357982) (end 147.843146 100.525128) (width 0.127) (layer "F.Cu") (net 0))
 (segment (start 152.439339 98.050253) (end 151.442 97.052914) (width 0.127) (layer "F.Cu") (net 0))
 (segment (start 151.244796 106.755204) (end 151 106.510408) (width 0.127) (layer "F.Cu") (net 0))
 (segment (start 155.678 93.75) (end 155.678 97.928) (width 0.127) (layer "F.Cu") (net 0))
 (segment (start 153.75 97.25) (end 152.854 96.354) (width 0.127) (layer "F.Cu") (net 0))
 (segment (start 156.75 110.25) (end 149.25 110.25) (width 0.127) (layer "F.Cu") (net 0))
 (segment (start 148.75 109.75) (end 148.75 108.810662) (width 0.127) (layer "F.Cu") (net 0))
 (segment (start 142.5 109.5) (end 147.353552 109.5) (width 0.127) (layer "F.Cu") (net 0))
 (segment (start 149.25 97.75) (end 150.03 96.97) (width 0.127) (layer "F.Cu") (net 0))
 (segment (start 147.146447 109) (end 147 109) (width 0.127) (layer "F.Cu") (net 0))
 (segment (start 157.796 93.75) (end 157.796 97.046) (width 0.127) (layer "F.Cu") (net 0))
 (segment (start 159.25 99.75) (end 159.25 98) (width 0.127) (layer "F.Cu") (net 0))
 (segment (start 137.85 104.85) (end 142.5 109.5) (width 0.127) (layer "F.Cu") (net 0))
 (segment (start 140.852 96.148) (end 140.852 93.75) (width 0.127) (layer "F.Cu") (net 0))
 (segment (start 139.75 97.554) (end 139.75 106) (width 0.127) (layer "F.Cu") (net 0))
 (segment (start 144.85 105.35) (end 143.6 105.35) (width 0.127) (layer "F.Cu") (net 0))
 (segment (start 143.676 93.75) (end 143.676 96.357982) (width 0.127) (layer "F.Cu") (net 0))
 (segment (start 159.208 93.75) (end 159.208 97.458) (width 0.127) (layer "F.Cu") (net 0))
 (segment (start 156.384 93.75) (end 156.384 100.469552) (width 0.127) (layer "F.Cu") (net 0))
 (segment (start 146.25 106.75) (end 144.85 105.35) (width 0.127) (layer "F.Cu") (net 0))
 (segment (start 145.489592 101) (end 141.25 101) (width 0.127) (layer "F.Cu") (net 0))
 (via (at 146.25 106.75) (size 0.6) (drill 0.3) (layers "F.Cu" "B.Cu") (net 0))
 (via (at 149 91.25) (size 0.6) (drill 0.3) (layers "F.Cu" "B.Cu") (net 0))
 (via (at 151 106.5) (size 0.6) (drill 0.3) (layers "F.Cu" "B.Cu") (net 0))
 (via (at 146 108) (size 0.6) (drill 0.3) (layers "F.Cu" "B.Cu") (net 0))
 (via (at 146.5 96.5) (size 0.6) (drill 0.3) (layers "F.Cu" "B.Cu") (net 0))
 (via (at 148.25 92) (size 0.6) (drill 0.3) (layers "F.Cu" "B.Cu") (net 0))
 (segment (start 149 91.25) (end 149 96.25) (width 0.127) (layer "B.Cu") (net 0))
 (segment (start 151 106.5) (end 147.714 103.214) (width 0.127) (layer "B.Cu") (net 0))
 (segment (start 152.1844 98.6284) (end 147.714 98.6284) (width 0.127) (layer "B.Cu") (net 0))
 (segment (start 148.25 94.75) (end 146.5 96.5) (width 0.127) (layer "B.Cu") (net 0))
 (segment (start 144.5 105.7404) (end 141.11 105.7404) (width 0.127) (layer "B.Cu") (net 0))
 (segment (start 147.714 103.214) (end 147.714 102.75) (width 0.127) (layer "B.Cu") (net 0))
 (segment (start 141.11 105.7404) (end 140.9576 105.588) (width 0.127) (layer "B.Cu") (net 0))
 (segment (start 147.714 105.286) (end 146.25 106.75) (width 0.127) (layer "B.Cu") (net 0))
 (segment (start 159.0424 107.9576) (end 156 111) (width 0.127) (layer "B.Cu") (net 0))
 (segment (start 145 107) (end 146 108) (width 0.127) (layer "B.Cu") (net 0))
 (segment (start 147.714 98.6284) (end 147.714 102.75) (width 0.127) (layer "B.Cu") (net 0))
 (segment (start 146 108) (end 149 111) (width 0.127) (layer "B.Cu") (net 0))
 (segment (start 149 111) (end 156 111) (width 0.127) (layer "B.Cu") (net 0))
 (segment (start 145 107) (end 145 106.2404) (width 0.127) (layer "B.Cu") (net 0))
 (segment (start 145 106.2404) (end 144.5 105.7404) (width 0.127) (layer "B.Cu") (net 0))
 (segment (start 148.25 92) (end 148.25 94.75) (width 0.127) (layer "B.Cu") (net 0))
 (segment (start 147.714 102.75) (end 147.714 105.286) (width 0.127) (layer "B.Cu") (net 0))
 (segment (start 147.714 97.536) (end 147.714 98.6284) (width 0.127) (layer "B.Cu") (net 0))
 (segment (start 159.0424 105.7404) (end 159.0424 107.9576) (width 0.127) (layer "B.Cu") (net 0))
 (segment (start 149 96.25) (end 147.714 97.536) (width 0.127) (layer "B.Cu") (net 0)))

